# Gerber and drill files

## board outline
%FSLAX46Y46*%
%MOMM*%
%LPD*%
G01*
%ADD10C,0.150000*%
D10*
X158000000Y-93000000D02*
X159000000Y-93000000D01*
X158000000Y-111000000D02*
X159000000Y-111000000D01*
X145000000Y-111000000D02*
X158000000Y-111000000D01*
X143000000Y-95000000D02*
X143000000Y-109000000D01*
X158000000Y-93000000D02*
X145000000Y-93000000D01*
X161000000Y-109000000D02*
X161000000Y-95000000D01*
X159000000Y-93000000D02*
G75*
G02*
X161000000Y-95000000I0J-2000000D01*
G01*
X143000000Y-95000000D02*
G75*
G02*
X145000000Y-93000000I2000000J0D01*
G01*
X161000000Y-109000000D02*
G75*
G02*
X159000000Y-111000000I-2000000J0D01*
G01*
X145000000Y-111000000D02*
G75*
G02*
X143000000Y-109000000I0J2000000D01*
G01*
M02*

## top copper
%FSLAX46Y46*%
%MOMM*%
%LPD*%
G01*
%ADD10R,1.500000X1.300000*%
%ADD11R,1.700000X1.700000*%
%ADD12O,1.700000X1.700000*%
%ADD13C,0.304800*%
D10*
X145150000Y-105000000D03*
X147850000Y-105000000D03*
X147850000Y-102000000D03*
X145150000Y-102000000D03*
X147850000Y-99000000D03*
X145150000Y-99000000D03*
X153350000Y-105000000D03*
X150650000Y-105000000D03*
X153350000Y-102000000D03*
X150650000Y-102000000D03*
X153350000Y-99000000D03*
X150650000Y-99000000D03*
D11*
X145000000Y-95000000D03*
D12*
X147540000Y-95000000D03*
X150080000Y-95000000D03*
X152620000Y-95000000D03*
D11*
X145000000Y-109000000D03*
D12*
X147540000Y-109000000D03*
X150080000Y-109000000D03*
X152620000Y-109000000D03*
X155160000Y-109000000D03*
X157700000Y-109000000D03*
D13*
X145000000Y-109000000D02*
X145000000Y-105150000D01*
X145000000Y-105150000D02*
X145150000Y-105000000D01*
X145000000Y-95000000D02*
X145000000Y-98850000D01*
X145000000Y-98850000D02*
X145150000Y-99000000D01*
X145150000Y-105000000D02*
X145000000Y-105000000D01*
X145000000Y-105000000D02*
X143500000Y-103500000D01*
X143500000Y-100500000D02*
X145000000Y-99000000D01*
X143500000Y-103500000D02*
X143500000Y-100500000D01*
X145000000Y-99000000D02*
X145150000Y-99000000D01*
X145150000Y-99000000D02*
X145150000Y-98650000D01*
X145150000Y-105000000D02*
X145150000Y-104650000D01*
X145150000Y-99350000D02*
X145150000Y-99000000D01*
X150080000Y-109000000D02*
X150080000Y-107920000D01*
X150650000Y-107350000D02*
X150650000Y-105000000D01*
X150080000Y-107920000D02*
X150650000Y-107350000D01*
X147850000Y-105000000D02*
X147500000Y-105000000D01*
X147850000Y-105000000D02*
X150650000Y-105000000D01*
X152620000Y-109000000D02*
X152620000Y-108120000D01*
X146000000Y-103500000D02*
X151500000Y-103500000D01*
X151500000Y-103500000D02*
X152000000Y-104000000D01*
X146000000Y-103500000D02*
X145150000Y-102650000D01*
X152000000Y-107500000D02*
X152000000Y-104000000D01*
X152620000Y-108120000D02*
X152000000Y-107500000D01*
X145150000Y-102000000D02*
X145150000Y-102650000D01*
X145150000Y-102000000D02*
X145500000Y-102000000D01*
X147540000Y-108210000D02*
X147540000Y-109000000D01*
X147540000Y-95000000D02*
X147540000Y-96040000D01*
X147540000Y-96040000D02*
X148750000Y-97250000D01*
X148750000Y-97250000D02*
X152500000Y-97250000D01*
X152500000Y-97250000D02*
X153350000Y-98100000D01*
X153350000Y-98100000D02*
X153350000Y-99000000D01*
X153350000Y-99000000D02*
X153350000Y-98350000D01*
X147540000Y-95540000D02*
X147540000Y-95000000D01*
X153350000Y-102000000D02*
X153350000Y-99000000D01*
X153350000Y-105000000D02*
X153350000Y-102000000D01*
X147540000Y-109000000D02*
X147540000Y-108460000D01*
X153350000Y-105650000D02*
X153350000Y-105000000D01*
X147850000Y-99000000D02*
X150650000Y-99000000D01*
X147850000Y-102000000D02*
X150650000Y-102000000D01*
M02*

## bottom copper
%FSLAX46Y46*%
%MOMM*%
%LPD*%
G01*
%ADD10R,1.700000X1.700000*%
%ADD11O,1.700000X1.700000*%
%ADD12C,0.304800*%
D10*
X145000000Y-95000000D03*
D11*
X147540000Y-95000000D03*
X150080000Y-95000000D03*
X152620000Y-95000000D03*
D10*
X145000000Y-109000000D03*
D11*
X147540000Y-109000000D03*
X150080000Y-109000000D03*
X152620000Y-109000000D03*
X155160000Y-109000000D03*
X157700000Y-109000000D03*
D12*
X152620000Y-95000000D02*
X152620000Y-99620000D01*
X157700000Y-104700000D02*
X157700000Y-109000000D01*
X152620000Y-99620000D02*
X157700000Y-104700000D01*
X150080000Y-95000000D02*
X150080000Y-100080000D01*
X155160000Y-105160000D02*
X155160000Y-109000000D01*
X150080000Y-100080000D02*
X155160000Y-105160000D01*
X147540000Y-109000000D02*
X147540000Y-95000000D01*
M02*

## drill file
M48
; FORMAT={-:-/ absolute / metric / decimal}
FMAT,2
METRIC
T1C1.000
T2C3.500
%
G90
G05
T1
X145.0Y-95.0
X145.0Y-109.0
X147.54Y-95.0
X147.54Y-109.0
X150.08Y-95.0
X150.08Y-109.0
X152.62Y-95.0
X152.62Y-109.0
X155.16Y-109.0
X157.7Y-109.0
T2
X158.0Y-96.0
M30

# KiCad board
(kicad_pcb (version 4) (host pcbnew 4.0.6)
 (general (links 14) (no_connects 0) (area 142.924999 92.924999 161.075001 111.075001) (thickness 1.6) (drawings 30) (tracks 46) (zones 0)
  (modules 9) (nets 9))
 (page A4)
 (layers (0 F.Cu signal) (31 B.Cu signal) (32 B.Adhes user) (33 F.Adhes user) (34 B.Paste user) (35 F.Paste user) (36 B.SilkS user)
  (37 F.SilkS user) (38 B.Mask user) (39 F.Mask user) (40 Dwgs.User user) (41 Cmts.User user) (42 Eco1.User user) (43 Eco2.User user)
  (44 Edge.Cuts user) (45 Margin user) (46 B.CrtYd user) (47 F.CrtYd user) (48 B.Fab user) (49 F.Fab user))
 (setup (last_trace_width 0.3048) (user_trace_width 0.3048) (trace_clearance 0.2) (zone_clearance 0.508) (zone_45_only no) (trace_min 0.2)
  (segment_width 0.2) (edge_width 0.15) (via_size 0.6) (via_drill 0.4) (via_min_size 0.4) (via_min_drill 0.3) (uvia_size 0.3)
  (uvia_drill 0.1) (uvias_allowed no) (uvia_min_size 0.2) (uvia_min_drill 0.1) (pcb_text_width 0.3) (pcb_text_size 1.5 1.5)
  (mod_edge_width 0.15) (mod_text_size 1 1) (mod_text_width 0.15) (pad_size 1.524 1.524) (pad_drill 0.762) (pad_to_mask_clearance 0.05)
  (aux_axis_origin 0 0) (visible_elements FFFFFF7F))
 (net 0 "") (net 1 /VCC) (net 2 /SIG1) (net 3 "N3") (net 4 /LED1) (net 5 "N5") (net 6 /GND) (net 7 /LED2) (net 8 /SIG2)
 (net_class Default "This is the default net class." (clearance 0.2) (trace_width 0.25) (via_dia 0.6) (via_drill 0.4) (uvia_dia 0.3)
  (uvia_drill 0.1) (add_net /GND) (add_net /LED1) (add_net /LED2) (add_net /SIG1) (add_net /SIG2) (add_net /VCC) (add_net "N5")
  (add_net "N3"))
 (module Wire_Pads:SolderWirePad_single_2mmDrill (layer F.Cu) (at 158 96)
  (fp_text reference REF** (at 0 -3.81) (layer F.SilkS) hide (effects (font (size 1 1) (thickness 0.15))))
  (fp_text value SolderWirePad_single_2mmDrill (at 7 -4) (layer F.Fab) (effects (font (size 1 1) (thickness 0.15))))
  (pad "" np_thru_hole circle (at 0 0) (size 3.5 3.5) (drill 3.5) (layers *.Cu *.Mask)))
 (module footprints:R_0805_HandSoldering (layer F.Cu) (at 146.5 105)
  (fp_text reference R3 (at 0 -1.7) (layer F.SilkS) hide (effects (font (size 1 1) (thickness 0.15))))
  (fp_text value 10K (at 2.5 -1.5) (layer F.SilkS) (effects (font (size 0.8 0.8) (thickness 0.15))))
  (pad 1 smd rect (at -1.35 0) (size 1.5 1.3) (layers F.Cu F.Paste F.Mask) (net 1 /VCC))
  (pad 2 smd rect (at 1.35 0) (size 1.5 1.3) (layers F.Cu F.Paste F.Mask) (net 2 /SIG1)))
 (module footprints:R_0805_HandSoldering (layer F.Cu) (at 146.5 102 180)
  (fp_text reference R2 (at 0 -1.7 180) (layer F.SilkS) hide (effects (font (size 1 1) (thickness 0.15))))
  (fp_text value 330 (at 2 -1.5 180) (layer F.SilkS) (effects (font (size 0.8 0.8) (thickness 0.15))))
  (pad 1 smd rect (at -1.35 0 180) (size 1.5 1.3) (layers F.Cu F.Paste F.Mask) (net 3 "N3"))
  (pad 2 smd rect (at 1.35 0 180) (size 1.5 1.3) (layers F.Cu F.Paste F.Mask) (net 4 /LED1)))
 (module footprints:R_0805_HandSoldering (layer F.Cu) (at 146.5 99 180)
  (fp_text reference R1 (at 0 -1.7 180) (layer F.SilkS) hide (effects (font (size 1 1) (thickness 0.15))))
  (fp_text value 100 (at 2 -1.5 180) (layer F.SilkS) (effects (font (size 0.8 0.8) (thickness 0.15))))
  (pad 1 smd rect (at -1.35 0 180) (size 1.5 1.3) (layers F.Cu F.Paste F.Mask) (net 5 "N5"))
  (pad 2 smd rect (at 1.35 0 180) (size 1.5 1.3) (layers F.Cu F.Paste F.Mask) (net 1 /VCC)))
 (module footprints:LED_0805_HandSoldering (layer F.Cu) (at 152 105 180)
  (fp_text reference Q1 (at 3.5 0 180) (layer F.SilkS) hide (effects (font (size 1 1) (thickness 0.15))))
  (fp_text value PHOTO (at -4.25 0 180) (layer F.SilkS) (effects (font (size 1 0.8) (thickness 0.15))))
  (pad 1 smd rect (at -1.35 0 180) (size 1.5 1.3) (layers F.Cu F.Paste F.Mask) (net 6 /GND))
  (pad 2 smd rect (at 1.35 0 180) (size 1.5 1.3) (layers F.Cu F.Paste F.Mask) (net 2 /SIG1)))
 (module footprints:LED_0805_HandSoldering (layer F.Cu) (at 152 102 180)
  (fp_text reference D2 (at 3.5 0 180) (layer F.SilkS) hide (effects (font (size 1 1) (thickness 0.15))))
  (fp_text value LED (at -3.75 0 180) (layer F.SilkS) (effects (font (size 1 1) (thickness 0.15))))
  (pad 1 smd rect (at -1.35 0 180) (size 1.5 1.3) (layers F.Cu F.Paste F.Mask) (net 6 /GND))
  (pad 2 smd rect (at 1.35 0 180) (size 1.5 1.3) (layers F.Cu F.Paste F.Mask) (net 3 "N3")))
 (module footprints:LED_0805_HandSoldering (layer F.Cu) (at 152 99 180)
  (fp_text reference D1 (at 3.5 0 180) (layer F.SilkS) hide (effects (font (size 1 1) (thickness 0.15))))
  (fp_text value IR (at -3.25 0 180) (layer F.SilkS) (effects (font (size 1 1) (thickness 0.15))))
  (pad 1 smd rect (at -1.35 0 180) (size 1.5 1.3) (layers F.Cu F.Paste F.Mask) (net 6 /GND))
  (pad 2 smd rect (at 1.35 0 180) (size 1.5 1.3) (layers F.Cu F.Paste F.Mask) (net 5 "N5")))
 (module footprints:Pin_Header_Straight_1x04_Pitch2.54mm (layer F.Cu) (at 145 95 90)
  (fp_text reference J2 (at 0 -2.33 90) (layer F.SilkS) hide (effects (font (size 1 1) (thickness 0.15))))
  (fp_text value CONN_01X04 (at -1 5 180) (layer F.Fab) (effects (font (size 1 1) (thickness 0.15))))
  (pad 1 thru_hole rect (at 0 0 90) (size 1.7 1.7) (drill 1) (layers *.Cu *.Mask) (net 1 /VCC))
  (pad 2 thru_hole oval (at 0 2.54 90) (size 1.7 1.7) (drill 1) (layers *.Cu *.Mask) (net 6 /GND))
  (pad 3 thru_hole oval (at 0 5.08 90) (size 1.7 1.7) (drill 1) (layers *.Cu *.Mask) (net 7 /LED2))
  (pad 4 thru_hole oval (at 0 7.62 90) (size 1.7 1.7) (drill 1) (layers *.Cu *.Mask) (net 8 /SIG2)))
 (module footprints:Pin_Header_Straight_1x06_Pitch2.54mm (layer F.Cu) (at 145 109 90)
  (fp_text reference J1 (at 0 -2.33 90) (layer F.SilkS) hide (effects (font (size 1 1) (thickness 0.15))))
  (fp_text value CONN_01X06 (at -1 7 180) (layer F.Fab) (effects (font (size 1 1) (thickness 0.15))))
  (pad 1 thru_hole rect (at 0 0 90) (size 1.7 1.7) (drill 1) (layers *.Cu *.Mask) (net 1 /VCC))
  (pad 2 thru_hole oval (at 0 2.54 90) (size 1.7 1.7) (drill 1) (layers *.Cu *.Mask) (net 6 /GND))
  (pad 3 thru_hole oval (at 0 5.08 90) (size 1.7 1.7) (drill 1) (layers *.Cu *.Mask) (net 2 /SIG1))
  (pad 4 thru_hole oval (at 0 7.62 90) (size 1.7 1.7) (drill 1) (layers *.Cu *.Mask) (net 4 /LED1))
  (pad 5 thru_hole oval (at 0 10.16 90) (size 1.7 1.7) (drill 1) (layers *.Cu *.Mask) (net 7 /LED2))
  (pad 6 thru_hole oval (at 0 12.7 90) (size 1.7 1.7) (drill 1) (layers *.Cu *.Mask) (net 8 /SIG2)))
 (gr_line (start 158 93) (end 159 93) (angle 90) (layer Edge.Cuts) (width 0.15))
 (gr_line (start 158 111) (end 159 111) (angle 90) (layer Edge.Cuts) (width 0.15))
 (gr_line (start 145 111) (end 158 111) (angle 90) (layer Edge.Cuts) (width 0.15))
 (gr_line (start 143 95) (end 143 109) (angle 90) (layer Edge.Cuts) (width 0.15))
 (gr_line (start 158 93) (end 145 93) (angle 90) (layer Edge.Cuts) (width 0.15))
 (gr_line (start 161 109) (end 161 95) (angle 90) (layer Edge.Cuts) (width 0.15))
 (gr_arc (start 159 95) (end 159 93) (angle 90) (layer Edge.Cuts) (width 0.15))
 (gr_arc (start 145 95) (end 143 95) (angle 90) (layer Edge.Cuts) (width 0.15))
 (gr_arc (start 159 109) (end 161 109) (angle 90) (layer Edge.Cuts) (width 0.15))
 (gr_arc (start 145 109) (end 145 111) (angle 90) (layer Edge.Cuts) (width 0.15))
 (segment (start 145 109) (end 145 105.15) (width 0.3048) (layer F.Cu) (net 1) (status C00000))
 (segment (start 145 105.15) (end 145.15 105) (width 0.3048) (layer F.Cu) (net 1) (status C00000))
 (segment (start 145 95) (end 145 98.85) (width 0.3048) (layer F.Cu) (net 1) (status C00000))
 (segment (start 145 98.85) (end 145.15 99) (width 0.3048) (layer F.Cu) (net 1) (status C00000))
 (segment (start 145.15 105) (end 145 105) (width 0.3048) (layer F.Cu) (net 1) (status C00000))
 (segment (start 145 105) (end 143.5 103.5) (width 0.3048) (layer F.Cu) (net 1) (status 400000))
 (segment (start 143.5 100.5) (end 145 99) (width 0.3048) (layer F.Cu) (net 1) (status 800000))
 (segment (start 143.5 103.5) (end 143.5 100.5) (width 0.3048) (layer F.Cu) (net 1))
 (segment (start 145 99) (end 145.15 99) (width 0.3048) (layer F.Cu) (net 1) (status C00000))
 (segment (start 145.15 99) (end 145.15 98.65) (width 0.3048) (layer F.Cu) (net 1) (status 30))
 (segment (start 145.15 105) (end 145.15 104.65) (width 0.3048) (layer F.Cu) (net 1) (status 30))
 (segment (start 145.15 99.35) (end 145.15 99) (width 0.3048) (layer F.Cu) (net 1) (status 30))
 (segment (start 150.08 109) (end 150.08 107.92) (width 0.3048) (layer F.Cu) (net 2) (status 400000))
 (segment (start 150.65 107.35) (end 150.65 105) (width 0.3048) (layer F.Cu) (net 2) (status 800000))
 (segment (start 150.08 107.92) (end 150.65 107.35) (width 0.3048) (layer F.Cu) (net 2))
 (segment (start 147.85 105) (end 147.5 105) (width 0.3048) (layer F.Cu) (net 2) (status 30))
 (segment (start 147.85 105) (end 150.65 105) (width 0.3048) (layer F.Cu) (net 2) (status 10))
 (segment (start 152.62 95) (end 152.62 99.62) (width 0.3048) (layer B.Cu) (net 8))
 (segment (start 157.7 104.7) (end 157.7 109) (width 0.3048) (layer B.Cu) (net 8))
 (segment (start 152.62 99.62) (end 157.7 104.7) (width 0.3048) (layer B.Cu) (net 8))
 (segment (start 152.62 109) (end 152.62 108.12) (width 0.3048) (layer F.Cu) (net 4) (status 400000))
 (segment (start 146 103.5) (end 151.5 103.5) (width 0.3048) (layer F.Cu) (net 4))
 (segment (start 151.5 103.5) (end 152 104) (width 0.3048) (layer F.Cu) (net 4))
 (segment (start 146 103.5) (end 145.15 102.65) (width 0.3048) (layer F.Cu) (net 4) (status 800000))
 (segment (start 152 107.5) (end 152 104) (width 0.3048) (layer F.Cu) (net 4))
 (segment (start 152.62 108.12) (end 152 107.5) (width 0.3048) (layer F.Cu) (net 4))
 (segment (start 145.15 102) (end 145.15 102.65) (width 0.3048) (layer F.Cu) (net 4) (status C00000))
 (segment (start 145.15 102) (end 145.5 102) (width 0.3048) (layer F.Cu) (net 4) (status 30))
 (segment (start 150.08 95) (end 150.08 100.08) (width 0.3048) (layer B.Cu) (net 7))
 (segment (start 155.16 105.16) (end 155.16 109) (width 0.3048) (layer B.Cu) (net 7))
 (segment (start 150.08 100.08) (end 155.16 105.16) (width 0.3048) (layer B.Cu) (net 7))
 (segment (start 147.54 109) (end 147.54 95) (width 0.3048) (layer B.Cu) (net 6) (status C00000))
 (segment (start 147.54 108.21) (end 147.54 109) (width 0.3048) (layer F.Cu) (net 6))
 (segment (start 147.54 95) (end 147.54 96.04) (width 0.3048) (layer F.Cu) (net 6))
 (segment (start 147.54 96.04) (end 148.75 97.25) (width 0.3048) (layer F.Cu) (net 6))
 (segment (start 148.75 97.25) (end 152.5 97.25) (width 0.3048) (layer F.Cu) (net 6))
 (segment (start 152.5 97.25) (end 153.35 98.1) (width 0.3048) (layer F.Cu) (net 6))
 (segment (start 153.35 98.1) (end 153.35 99) (width 0.3048) (layer F.Cu) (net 6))
 (segment (start 153.35 99) (end 153.35 98.35) (width 0.3048) (layer F.Cu) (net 6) (status 30))
 (segment (start 147.54 95.54) (end 147.54 95) (width 0.3048) (layer F.Cu) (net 6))
 (segment (start 153.35 102) (end 153.35 99) (width 0.3048) (layer F.Cu) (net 6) (status 20))
 (segment (start 153.35 105) (end 153.35 102) (width 0.3048) (layer F.Cu) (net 6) (status 10))
 (segment (start 147.54 109) (end 147.54 108.46) (width 0.3048) (layer F.Cu) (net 6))
 (segment (start 153.35 105.65) (end 153.35 105) (width 0.3048) (layer F.Cu) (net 6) (status 30))
 (segment (start 147.85 99) (end 150.65 99) (width 0.3048) (layer F.Cu) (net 5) (status 10))
 (segment (start 147.85 102) (end 150.65 102) (width 0.3048) (layer F.Cu) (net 3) (status 10)))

